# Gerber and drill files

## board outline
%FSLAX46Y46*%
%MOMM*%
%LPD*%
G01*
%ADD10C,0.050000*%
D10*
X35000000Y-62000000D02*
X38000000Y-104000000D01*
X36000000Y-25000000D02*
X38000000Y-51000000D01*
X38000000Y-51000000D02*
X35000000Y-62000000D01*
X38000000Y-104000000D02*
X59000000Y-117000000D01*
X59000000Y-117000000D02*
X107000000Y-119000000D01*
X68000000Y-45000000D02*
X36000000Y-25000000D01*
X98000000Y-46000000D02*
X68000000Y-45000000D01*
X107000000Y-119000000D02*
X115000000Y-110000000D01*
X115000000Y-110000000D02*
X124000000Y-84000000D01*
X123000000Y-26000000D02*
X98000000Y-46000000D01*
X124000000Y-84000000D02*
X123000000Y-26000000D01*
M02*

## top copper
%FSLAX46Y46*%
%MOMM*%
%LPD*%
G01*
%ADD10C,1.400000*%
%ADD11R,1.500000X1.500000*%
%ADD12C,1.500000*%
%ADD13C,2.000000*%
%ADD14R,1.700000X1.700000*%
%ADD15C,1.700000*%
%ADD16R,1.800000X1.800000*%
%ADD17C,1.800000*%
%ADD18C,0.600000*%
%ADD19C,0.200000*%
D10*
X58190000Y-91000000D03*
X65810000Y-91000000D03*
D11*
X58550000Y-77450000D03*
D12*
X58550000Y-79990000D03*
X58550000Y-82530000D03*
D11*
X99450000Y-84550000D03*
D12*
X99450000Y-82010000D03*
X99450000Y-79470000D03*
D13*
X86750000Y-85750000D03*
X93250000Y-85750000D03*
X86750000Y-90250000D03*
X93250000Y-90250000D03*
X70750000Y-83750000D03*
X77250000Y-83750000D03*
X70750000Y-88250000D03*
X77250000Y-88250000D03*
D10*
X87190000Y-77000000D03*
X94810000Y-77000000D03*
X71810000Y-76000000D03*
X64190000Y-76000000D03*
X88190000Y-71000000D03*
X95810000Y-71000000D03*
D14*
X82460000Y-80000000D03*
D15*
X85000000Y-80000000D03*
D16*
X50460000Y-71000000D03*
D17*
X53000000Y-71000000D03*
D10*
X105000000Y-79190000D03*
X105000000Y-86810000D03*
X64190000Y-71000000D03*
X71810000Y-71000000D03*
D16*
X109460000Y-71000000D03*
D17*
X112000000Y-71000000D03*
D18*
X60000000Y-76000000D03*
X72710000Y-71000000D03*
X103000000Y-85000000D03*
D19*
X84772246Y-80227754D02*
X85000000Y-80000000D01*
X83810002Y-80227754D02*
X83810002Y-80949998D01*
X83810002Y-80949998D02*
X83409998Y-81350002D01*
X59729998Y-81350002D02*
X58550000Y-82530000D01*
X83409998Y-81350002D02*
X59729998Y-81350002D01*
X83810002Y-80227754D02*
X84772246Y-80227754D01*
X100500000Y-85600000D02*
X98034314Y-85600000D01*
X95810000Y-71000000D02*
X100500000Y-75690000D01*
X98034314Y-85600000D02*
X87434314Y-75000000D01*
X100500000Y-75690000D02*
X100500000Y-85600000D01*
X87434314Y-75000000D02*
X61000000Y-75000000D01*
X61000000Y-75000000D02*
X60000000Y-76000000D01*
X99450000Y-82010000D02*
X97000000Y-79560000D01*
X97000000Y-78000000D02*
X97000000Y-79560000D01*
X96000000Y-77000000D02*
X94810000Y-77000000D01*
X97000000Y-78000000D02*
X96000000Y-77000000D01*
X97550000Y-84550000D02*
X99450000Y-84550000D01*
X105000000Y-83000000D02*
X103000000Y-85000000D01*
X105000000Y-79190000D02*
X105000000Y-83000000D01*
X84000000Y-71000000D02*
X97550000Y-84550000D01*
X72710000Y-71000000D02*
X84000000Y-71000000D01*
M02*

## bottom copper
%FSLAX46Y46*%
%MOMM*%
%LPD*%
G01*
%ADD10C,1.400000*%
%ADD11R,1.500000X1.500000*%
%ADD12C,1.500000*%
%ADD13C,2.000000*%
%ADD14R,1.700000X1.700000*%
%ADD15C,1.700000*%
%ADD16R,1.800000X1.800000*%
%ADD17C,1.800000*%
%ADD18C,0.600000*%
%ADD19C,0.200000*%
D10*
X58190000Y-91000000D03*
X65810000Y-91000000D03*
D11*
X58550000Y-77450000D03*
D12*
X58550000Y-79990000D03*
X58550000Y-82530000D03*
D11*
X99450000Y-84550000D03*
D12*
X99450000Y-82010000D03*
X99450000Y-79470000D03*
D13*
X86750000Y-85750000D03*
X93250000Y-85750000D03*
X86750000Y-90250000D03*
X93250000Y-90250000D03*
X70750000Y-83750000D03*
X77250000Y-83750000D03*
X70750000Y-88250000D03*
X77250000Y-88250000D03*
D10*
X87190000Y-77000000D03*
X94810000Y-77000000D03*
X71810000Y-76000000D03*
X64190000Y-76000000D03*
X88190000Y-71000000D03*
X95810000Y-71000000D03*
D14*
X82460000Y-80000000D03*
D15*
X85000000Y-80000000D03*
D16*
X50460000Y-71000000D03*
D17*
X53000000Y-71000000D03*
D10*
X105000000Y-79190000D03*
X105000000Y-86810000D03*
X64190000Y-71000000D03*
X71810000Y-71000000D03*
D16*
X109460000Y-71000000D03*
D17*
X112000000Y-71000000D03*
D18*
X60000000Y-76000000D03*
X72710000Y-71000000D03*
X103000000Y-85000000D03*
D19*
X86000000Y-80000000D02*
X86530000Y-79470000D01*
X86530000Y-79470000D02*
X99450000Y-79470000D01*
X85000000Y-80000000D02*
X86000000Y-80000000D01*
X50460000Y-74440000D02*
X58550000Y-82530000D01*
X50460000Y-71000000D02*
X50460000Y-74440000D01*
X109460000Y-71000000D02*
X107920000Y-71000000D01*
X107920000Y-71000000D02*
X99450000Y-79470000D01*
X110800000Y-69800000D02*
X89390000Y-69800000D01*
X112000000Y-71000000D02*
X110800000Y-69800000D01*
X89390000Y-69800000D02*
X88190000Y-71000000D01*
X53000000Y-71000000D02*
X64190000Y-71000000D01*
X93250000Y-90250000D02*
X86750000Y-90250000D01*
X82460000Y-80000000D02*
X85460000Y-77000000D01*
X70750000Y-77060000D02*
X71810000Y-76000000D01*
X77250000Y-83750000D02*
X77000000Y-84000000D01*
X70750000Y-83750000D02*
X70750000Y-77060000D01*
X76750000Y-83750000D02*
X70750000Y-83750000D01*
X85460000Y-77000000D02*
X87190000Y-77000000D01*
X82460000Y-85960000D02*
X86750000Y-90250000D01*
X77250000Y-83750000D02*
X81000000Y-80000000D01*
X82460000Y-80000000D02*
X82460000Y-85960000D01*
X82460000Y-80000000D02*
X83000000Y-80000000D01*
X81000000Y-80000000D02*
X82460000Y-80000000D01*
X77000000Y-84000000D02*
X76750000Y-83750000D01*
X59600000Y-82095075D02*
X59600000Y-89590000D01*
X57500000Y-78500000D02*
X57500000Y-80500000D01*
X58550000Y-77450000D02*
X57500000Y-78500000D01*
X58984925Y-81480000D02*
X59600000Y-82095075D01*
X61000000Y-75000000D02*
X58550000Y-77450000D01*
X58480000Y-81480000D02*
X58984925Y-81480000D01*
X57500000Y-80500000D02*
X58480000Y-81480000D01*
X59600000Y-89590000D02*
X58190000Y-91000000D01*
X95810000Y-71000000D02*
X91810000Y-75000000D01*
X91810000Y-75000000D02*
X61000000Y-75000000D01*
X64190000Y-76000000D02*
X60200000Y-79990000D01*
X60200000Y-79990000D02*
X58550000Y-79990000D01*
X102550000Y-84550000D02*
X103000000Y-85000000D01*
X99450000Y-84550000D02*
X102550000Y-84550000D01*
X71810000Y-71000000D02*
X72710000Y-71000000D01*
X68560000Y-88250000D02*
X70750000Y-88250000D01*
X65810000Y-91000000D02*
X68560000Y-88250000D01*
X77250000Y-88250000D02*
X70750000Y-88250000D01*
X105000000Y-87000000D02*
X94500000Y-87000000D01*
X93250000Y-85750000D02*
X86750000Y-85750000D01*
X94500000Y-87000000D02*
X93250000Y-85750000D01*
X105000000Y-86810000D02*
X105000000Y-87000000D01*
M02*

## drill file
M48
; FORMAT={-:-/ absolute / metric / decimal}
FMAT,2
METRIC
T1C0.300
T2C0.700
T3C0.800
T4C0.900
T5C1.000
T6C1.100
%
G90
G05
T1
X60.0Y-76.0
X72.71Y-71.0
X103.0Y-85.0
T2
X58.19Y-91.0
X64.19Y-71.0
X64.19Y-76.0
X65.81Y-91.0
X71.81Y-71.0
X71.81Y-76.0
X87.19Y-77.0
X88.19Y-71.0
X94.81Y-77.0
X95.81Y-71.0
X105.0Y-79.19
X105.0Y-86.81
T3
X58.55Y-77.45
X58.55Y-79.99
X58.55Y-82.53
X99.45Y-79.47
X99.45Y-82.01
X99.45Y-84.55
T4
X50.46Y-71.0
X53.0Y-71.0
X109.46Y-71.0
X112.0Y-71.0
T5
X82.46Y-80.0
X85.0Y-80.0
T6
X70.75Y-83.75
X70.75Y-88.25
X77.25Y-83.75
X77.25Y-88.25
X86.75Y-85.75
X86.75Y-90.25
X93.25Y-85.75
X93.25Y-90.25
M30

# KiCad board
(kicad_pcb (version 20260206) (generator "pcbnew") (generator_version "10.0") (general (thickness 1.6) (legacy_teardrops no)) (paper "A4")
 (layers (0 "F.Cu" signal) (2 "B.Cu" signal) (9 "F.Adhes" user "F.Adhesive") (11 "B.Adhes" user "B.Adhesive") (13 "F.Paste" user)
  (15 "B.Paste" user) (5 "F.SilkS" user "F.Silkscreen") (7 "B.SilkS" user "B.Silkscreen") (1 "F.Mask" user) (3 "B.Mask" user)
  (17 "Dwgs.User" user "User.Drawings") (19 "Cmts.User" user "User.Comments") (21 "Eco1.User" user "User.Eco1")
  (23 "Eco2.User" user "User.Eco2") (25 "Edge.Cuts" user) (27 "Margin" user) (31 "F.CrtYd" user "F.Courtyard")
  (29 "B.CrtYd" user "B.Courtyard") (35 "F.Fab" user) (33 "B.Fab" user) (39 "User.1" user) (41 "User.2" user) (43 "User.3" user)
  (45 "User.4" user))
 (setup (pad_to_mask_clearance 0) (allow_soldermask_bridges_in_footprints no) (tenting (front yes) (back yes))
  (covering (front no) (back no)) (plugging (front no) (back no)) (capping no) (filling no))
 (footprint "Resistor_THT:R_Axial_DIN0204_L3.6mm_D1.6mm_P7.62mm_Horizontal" (layer "F.Cu") (at 58.19 91)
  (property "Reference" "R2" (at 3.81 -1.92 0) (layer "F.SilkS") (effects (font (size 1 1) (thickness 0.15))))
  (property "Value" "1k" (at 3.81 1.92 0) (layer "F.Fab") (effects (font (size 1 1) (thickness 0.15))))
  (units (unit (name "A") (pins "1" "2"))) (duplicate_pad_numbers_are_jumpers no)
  (pad "1" thru_hole circle (at 0 0) (size 1.4 1.4) (drill 0.7) (layers "*.Cu" "*.Mask") (remove_unused_layers no) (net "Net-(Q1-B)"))
  (pad "2" thru_hole circle (at 7.62 0) (size 1.4 1.4) (drill 0.7) (layers "*.Cu" "*.Mask") (remove_unused_layers no) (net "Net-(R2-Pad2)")))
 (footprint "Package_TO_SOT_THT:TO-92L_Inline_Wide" (layer "F.Cu") (at 58.55 77.45 -90)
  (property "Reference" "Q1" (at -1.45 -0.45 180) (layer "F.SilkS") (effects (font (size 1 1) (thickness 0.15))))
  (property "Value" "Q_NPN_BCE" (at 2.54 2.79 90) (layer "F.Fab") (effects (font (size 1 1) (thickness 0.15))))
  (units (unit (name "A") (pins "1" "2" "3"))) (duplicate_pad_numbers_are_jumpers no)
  (pad "1" thru_hole rect (at 0 0 270) (size 1.5 1.5) (drill 0.8) (layers "*.Cu" "*.Mask") (remove_unused_layers no) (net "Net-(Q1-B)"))
  (pad "2" thru_hole circle (at 2.54 0 270) (size 1.5 1.5) (drill 0.8) (layers "*.Cu" "*.Mask") (remove_unused_layers no) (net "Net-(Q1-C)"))
  (pad "3" thru_hole circle (at 5.08 0 270) (size 1.5 1.5) (drill 0.8) (layers "*.Cu" "*.Mask") (remove_unused_layers no) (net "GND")))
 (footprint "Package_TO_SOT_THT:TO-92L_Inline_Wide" (layer "F.Cu") (at 99.45 84.55 90)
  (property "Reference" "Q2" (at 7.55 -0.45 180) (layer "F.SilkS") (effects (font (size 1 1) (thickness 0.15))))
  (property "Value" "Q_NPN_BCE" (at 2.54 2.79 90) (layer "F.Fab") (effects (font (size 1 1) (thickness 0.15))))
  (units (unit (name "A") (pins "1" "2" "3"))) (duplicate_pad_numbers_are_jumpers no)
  (pad "1" thru_hole rect (at 0 0 90) (size 1.5 1.5) (drill 0.8) (layers "*.Cu" "*.Mask") (remove_unused_layers no) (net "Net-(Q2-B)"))
  (pad "2" thru_hole circle (at 2.54 0 90) (size 1.5 1.5) (drill 0.8) (layers "*.Cu" "*.Mask") (remove_unused_layers no) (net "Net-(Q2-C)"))
  (pad "3" thru_hole circle (at 5.08 0 90) (size 1.5 1.5) (drill 0.8) (layers "*.Cu" "*.Mask") (remove_unused_layers no) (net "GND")))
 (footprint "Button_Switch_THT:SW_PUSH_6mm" (layer "F.Cu") (at 86.75 85.75)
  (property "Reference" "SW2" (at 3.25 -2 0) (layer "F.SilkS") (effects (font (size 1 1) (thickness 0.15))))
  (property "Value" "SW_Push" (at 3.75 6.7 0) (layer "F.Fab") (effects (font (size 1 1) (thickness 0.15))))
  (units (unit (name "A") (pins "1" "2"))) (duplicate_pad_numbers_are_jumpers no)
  (pad "1" thru_hole circle (at 0 0 90) (size 2 2) (drill 1.1) (layers "*.Cu" "*.Mask") (remove_unused_layers no) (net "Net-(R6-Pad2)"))
  (pad "1" thru_hole circle (at 6.5 0 90) (size 2 2) (drill 1.1) (layers "*.Cu" "*.Mask") (remove_unused_layers no) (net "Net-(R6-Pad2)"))
  (pad "2" thru_hole circle (at 0 4.5 90) (size 2 2) (drill 1.1) (layers "*.Cu" "*.Mask") (remove_unused_layers no) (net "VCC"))
  (pad "2" thru_hole circle (at 6.5 4.5 90) (size 2 2) (drill 1.1) (layers "*.Cu" "*.Mask") (remove_unused_layers no) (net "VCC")))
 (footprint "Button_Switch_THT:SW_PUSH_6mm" (layer "F.Cu") (at 70.75 83.75)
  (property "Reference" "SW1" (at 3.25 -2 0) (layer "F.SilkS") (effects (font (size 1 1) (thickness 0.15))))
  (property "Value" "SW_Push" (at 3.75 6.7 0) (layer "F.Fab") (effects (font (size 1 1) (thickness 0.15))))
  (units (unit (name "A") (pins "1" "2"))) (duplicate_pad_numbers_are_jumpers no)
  (pad "1" thru_hole circle (at 0 0 90) (size 2 2) (drill 1.1) (layers "*.Cu" "*.Mask") (remove_unused_layers no) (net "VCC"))
  (pad "1" thru_hole circle (at 6.5 0 90) (size 2 2) (drill 1.1) (layers "*.Cu" "*.Mask") (remove_unused_layers no) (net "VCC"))
  (pad "2" thru_hole circle (at 0 4.5 90) (size 2 2) (drill 1.1) (layers "*.Cu" "*.Mask") (remove_unused_layers no) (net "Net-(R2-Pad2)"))
  (pad "2" thru_hole circle (at 6.5 4.5 90) (size 2 2) (drill 1.1) (layers "*.Cu" "*.Mask") (remove_unused_layers no) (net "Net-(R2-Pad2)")))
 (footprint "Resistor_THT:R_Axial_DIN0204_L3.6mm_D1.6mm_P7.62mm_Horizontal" (layer "F.Cu") (at 87.19 77)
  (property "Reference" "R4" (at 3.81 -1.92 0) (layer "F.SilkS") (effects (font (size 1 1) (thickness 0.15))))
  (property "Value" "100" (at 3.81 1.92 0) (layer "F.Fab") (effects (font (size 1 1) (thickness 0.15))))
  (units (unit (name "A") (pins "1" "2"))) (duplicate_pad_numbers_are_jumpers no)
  (pad "1" thru_hole circle (at 0 0) (size 1.4 1.4) (drill 0.7) (layers "*.Cu" "*.Mask") (remove_unused_layers no) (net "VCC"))
  (pad "2" thru_hole circle (at 7.62 0) (size 1.4 1.4) (drill 0.7) (layers "*.Cu" "*.Mask") (remove_unused_layers no) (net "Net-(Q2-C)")))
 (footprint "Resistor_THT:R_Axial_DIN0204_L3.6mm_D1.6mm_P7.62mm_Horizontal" (layer "F.Cu") (at 71.81 76 180)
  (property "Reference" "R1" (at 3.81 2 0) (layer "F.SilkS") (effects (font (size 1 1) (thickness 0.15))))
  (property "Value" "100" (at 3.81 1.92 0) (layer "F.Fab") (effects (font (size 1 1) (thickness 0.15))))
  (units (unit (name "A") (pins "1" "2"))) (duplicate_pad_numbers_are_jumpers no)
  (pad "1" thru_hole circle (at 0 0 180) (size 1.4 1.4) (drill 0.7) (layers "*.Cu" "*.Mask") (remove_unused_layers no) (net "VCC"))
  (pad "2" thru_hole circle (at 7.62 0 180) (size 1.4 1.4) (drill 0.7) (layers "*.Cu" "*.Mask") (remove_unused_layers no) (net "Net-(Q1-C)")))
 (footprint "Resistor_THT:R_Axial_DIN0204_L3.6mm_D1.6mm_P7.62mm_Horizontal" (layer "F.Cu") (at 88.19 71)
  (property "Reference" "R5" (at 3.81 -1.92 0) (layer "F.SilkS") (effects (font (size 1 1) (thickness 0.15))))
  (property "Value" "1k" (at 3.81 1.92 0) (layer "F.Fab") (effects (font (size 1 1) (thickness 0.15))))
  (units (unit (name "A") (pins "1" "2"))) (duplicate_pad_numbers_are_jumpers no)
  (pad "1" thru_hole circle (at 0 0) (size 1.4 1.4) (drill 0.7) (layers "*.Cu" "*.Mask") (remove_unused_layers no) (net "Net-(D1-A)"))
  (pad "2" thru_hole circle (at 7.62 0) (size 1.4 1.4) (drill 0.7) (layers "*.Cu" "*.Mask") (remove_unused_layers no) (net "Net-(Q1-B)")))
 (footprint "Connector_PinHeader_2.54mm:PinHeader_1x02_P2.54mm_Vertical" (layer "F.Cu") (at 82.46 80 90)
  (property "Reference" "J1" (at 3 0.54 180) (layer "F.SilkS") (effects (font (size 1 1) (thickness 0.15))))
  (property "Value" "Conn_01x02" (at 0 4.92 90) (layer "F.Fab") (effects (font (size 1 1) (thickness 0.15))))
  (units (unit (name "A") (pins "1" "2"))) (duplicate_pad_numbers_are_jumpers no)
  (pad "1" thru_hole rect (at 0 0 90) (size 1.7 1.7) (drill 1) (layers "*.Cu" "*.Mask") (remove_unused_layers no) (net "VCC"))
  (pad "2" thru_hole circle (at 0 2.54 90) (size 1.7 1.7) (drill 1) (layers "*.Cu" "*.Mask") (remove_unused_layers no) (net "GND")))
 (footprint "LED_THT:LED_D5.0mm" (layer "F.Cu") (at 50.46 71)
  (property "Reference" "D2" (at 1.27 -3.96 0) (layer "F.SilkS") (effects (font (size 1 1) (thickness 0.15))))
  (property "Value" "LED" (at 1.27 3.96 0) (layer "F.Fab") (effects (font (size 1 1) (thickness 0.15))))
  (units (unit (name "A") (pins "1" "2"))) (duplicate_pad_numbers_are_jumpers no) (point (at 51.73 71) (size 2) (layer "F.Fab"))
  (pad "1" thru_hole rect (at 0 0) (size 1.8 1.8) (drill 0.9) (layers "*.Cu" "*.Mask") (remove_unused_layers no) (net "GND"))
  (pad "2" thru_hole circle (at 2.54 0) (size 1.8 1.8) (drill 0.9) (layers "*.Cu" "*.Mask") (remove_unused_layers no) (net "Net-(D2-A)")))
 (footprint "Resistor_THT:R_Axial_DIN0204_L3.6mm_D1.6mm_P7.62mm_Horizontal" (layer "F.Cu") (at 105 79.19 -90)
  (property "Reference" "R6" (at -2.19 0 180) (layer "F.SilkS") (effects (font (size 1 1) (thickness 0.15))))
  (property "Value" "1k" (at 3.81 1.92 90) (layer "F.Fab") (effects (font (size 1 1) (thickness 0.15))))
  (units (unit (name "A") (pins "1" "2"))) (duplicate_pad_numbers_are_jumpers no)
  (pad "1" thru_hole circle (at 0 0 270) (size 1.4 1.4) (drill 0.7) (layers "*.Cu" "*.Mask") (remove_unused_layers no) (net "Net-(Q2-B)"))
  (pad "2" thru_hole circle (at 7.62 0 270) (size 1.4 1.4) (drill 0.7) (layers "*.Cu" "*.Mask") (remove_unused_layers no)
   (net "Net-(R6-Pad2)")))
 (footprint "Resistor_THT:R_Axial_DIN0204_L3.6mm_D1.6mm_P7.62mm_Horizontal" (layer "F.Cu") (at 64.19 71)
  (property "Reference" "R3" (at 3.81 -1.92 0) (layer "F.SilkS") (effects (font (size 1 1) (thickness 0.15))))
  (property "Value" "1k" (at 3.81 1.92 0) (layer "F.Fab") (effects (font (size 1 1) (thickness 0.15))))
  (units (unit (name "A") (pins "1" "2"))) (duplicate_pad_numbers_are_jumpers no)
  (pad "1" thru_hole circle (at 0 0) (size 1.4 1.4) (drill 0.7) (layers "*.Cu" "*.Mask") (remove_unused_layers no) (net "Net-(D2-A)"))
  (pad "2" thru_hole circle (at 7.62 0) (size 1.4 1.4) (drill 0.7) (layers "*.Cu" "*.Mask") (remove_unused_layers no) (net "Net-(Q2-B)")))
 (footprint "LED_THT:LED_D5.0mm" (layer "F.Cu") (at 109.46 71)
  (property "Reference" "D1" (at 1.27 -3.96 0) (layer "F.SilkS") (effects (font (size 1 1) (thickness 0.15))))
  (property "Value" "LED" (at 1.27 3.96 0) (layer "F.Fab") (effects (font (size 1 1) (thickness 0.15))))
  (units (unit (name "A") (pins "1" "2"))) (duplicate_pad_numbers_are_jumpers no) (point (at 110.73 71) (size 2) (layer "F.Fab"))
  (pad "1" thru_hole rect (at 0 0) (size 1.8 1.8) (drill 0.9) (layers "*.Cu" "*.Mask") (remove_unused_layers no) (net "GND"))
  (pad "2" thru_hole circle (at 2.54 0) (size 1.8 1.8) (drill 0.9) (layers "*.Cu" "*.Mask") (remove_unused_layers no) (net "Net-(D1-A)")))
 (gr_line (start 35 62) (end 38 104) (stroke (width 0.05) (type default)) (layer "Edge.Cuts"))
 (gr_line (start 36 25) (end 38 51) (stroke (width 0.05) (type default)) (layer "Edge.Cuts"))
 (gr_line (start 38 51) (end 35 62) (stroke (width 0.05) (type default)) (layer "Edge.Cuts"))
 (gr_line (start 38 104) (end 59 117) (stroke (width 0.05) (type default)) (layer "Edge.Cuts"))
 (gr_line (start 59 117) (end 107 119) (stroke (width 0.05) (type default)) (layer "Edge.Cuts"))
 (gr_line (start 68 45) (end 36 25) (stroke (width 0.05) (type default)) (layer "Edge.Cuts"))
 (gr_line (start 98 46) (end 68 45) (stroke (width 0.05) (type default)) (layer "Edge.Cuts"))
 (gr_line (start 107 119) (end 115 110) (stroke (width 0.05) (type default)) (layer "Edge.Cuts"))
 (gr_line (start 115 110) (end 124 84) (stroke (width 0.05) (type default)) (layer "Edge.Cuts"))
 (gr_line (start 123 26) (end 98 46) (stroke (width 0.05) (type default)) (layer "Edge.Cuts"))
 (gr_line (start 124 84) (end 123 26) (stroke (width 0.05) (type default)) (layer "Edge.Cuts"))
 (segment (start 84.772246 80.227754) (end 85 80) (width 0.2) (layer "F.Cu") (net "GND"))
 (segment (start 83.810002 80.227754) (end 83.810002 80.949998) (width 0.2) (layer "F.Cu") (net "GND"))
 (segment (start 83.810002 80.949998) (end 83.409998 81.350002) (width 0.2) (layer "F.Cu") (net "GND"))
 (segment (start 59.729998 81.350002) (end 58.55 82.53) (width 0.2) (layer "F.Cu") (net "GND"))
 (segment (start 83.409998 81.350002) (end 59.729998 81.350002) (width 0.2) (layer "F.Cu") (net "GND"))
 (segment (start 83.810002 80.227754) (end 84.772246 80.227754) (width 0.2) (layer "F.Cu") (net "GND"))
 (segment (start 86 80) (end 86.53 79.47) (width 0.2) (layer "B.Cu") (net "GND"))
 (segment (start 86.53 79.47) (end 99.45 79.47) (width 0.2) (layer "B.Cu") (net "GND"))
 (segment (start 85 80) (end 86 80) (width 0.2) (layer "B.Cu") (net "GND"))
 (segment (start 50.46 74.44) (end 58.55 82.53) (width 0.2) (layer "B.Cu") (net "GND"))
 (segment (start 50.46 71) (end 50.46 74.44) (width 0.2) (layer "B.Cu") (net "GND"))
 (segment (start 109.46 71) (end 107.92 71) (width 0.2) (layer "B.Cu") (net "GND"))
 (segment (start 107.92 71) (end 99.45 79.47) (width 0.2) (layer "B.Cu") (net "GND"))
 (segment (start 110.8 69.8) (end 89.39 69.8) (width 0.2) (layer "B.Cu") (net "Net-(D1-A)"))
 (segment (start 112 71) (end 110.8 69.8) (width 0.2) (layer "B.Cu") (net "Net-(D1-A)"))
 (segment (start 89.39 69.8) (end 88.19 71) (width 0.2) (layer "B.Cu") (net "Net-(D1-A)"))
 (segment (start 53 71) (end 64.19 71) (width 0.2) (layer "B.Cu") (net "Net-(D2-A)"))
 (segment (start 93.25 90.25) (end 86.75 90.25) (width 0.2) (layer "B.Cu") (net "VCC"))
 (segment (start 82.46 80) (end 85.46 77) (width 0.2) (layer "B.Cu") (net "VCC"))
 (segment (start 70.75 77.06) (end 71.81 76) (width 0.2) (layer "B.Cu") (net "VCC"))
 (segment (start 77.25 83.75) (end 77 84) (width 0.2) (layer "B.Cu") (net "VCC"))
 (segment (start 70.75 83.75) (end 70.75 77.06) (width 0.2) (layer "B.Cu") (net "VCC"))
 (segment (start 76.75 83.75) (end 70.75 83.75) (width 0.2) (layer "B.Cu") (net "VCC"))
 (segment (start 85.46 77) (end 87.19 77) (width 0.2) (layer "B.Cu") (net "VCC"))
 (segment (start 82.46 85.96) (end 86.75 90.25) (width 0.2) (layer "B.Cu") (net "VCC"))
 (segment (start 77.25 83.75) (end 81 80) (width 0.2) (layer "B.Cu") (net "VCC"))
 (segment (start 82.46 80) (end 82.46 85.96) (width 0.2) (layer "B.Cu") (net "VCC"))
 (segment (start 82.46 80) (end 83 80) (width 0.2) (layer "B.Cu") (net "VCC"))
 (segment (start 81 80) (end 82.46 80) (width 0.2) (layer "B.Cu") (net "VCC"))
 (segment (start 77 84) (end 76.75 83.75) (width 0.2) (layer "B.Cu") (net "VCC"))
 (segment (start 100.5 85.6) (end 98.034314 85.6) (width 0.2) (layer "F.Cu") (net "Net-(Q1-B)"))
 (segment (start 95.81 71) (end 100.5 75.69) (width 0.2) (layer "F.Cu") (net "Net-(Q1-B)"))
 (segment (start 98.034314 85.6) (end 87.434314 75) (width 0.2) (layer "F.Cu") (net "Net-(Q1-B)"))
 (segment (start 100.5 75.69) (end 100.5 85.6) (width 0.2) (layer "F.Cu") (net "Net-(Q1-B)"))
 (segment (start 87.434314 75) (end 61 75) (width 0.2) (layer "F.Cu") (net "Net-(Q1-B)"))
 (segment (start 61 75) (end 60 76) (width 0.2) (layer "F.Cu") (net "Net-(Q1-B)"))
 (via (at 60 76) (size 0.6) (drill 0.3) (layers "F.Cu" "B.Cu") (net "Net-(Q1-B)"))
 (segment (start 59.6 82.095075) (end 59.6 89.59) (width 0.2) (layer "B.Cu") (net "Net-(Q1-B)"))
 (segment (start 57.5 78.5) (end 57.5 80.5) (width 0.2) (layer "B.Cu") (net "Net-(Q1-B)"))
 (segment (start 58.55 77.45) (end 57.5 78.5) (width 0.2) (layer "B.Cu") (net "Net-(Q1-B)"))
 (segment (start 58.984925 81.48) (end 59.6 82.095075) (width 0.2) (layer "B.Cu") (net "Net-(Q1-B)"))
 (segment (start 61 75) (end 58.55 77.45) (width 0.2) (layer "B.Cu") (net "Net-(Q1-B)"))
 (segment (start 58.48 81.48) (end 58.984925 81.48) (width 0.2) (layer "B.Cu") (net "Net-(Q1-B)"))
 (segment (start 57.5 80.5) (end 58.48 81.48) (width 0.2) (layer "B.Cu") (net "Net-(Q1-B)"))
 (segment (start 59.6 89.59) (end 58.19 91) (width 0.2) (layer "B.Cu") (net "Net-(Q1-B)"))
 (segment (start 95.81 71) (end 91.81 75) (width 0.2) (layer "B.Cu") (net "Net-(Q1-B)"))
 (segment (start 91.81 75) (end 61 75) (width 0.2) (layer "B.Cu") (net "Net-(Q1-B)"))
 (segment (start 64.19 76) (end 60.2 79.99) (width 0.2) (layer "B.Cu") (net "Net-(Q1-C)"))
 (segment (start 60.2 79.99) (end 58.55 79.99) (width 0.2) (layer "B.Cu") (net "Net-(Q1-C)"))
 (segment (start 99.45 82.01) (end 97 79.56) (width 0.2) (layer "F.Cu") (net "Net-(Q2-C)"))
 (segment (start 97 78) (end 97 79.56) (width 0.2) (layer "F.Cu") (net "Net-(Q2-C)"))
 (segment (start 96 77) (end 94.81 77) (width 0.2) (layer "F.Cu") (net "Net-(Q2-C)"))
 (segment (start 97 78) (end 96 77) (width 0.2) (layer "F.Cu") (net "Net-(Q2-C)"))
 (segment (start 97.55 84.55) (end 99.45 84.55) (width 0.2) (layer "F.Cu") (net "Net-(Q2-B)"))
 (segment (start 105 83) (end 103 85) (width 0.2) (layer "F.Cu") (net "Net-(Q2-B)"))
 (segment (start 105 79.19) (end 105 83) (width 0.2) (layer "F.Cu") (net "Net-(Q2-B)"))
 (segment (start 84 71) (end 97.55 84.55) (width 0.2) (layer "F.Cu") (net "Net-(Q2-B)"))
 (segment (start 72.71 71) (end 84 71) (width 0.2) (layer "F.Cu") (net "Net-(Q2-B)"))
 (via (at 72.71 71) (size 0.6) (drill 0.3) (layers "F.Cu" "B.Cu") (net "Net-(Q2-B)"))
 (via (at 103 85) (size 0.6) (drill 0.3) (layers "F.Cu" "B.Cu") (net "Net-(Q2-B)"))
 (segment (start 102.55 84.55) (end 103 85) (width 0.2) (layer "B.Cu") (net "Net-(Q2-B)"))
 (segment (start 99.45 84.55) (end 102.55 84.55) (width 0.2) (layer "B.Cu") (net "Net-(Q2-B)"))
 (segment (start 71.81 71) (end 72.71 71) (width 0.2) (layer "B.Cu") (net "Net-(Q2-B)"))
 (segment (start 68.56 88.25) (end 70.75 88.25) (width 0.2) (layer "B.Cu") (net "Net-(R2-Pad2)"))
 (segment (start 65.81 91) (end 68.56 88.25) (width 0.2) (layer "B.Cu") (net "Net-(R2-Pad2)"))
 (segment (start 77.25 88.25) (end 70.75 88.25) (width 0.2) (layer "B.Cu") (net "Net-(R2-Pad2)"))
 (segment (start 105 87) (end 94.5 87) (width 0.2) (layer "B.Cu") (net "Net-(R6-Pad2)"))
 (segment (start 93.25 85.75) (end 86.75 85.75) (width 0.2) (layer "B.Cu") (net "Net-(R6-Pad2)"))
 (segment (start 94.5 87) (end 93.25 85.75) (width 0.2) (layer "B.Cu") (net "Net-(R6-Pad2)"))
 (segment (start 105 86.81) (end 105 87) (width 0.2) (layer "B.Cu") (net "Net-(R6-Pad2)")))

